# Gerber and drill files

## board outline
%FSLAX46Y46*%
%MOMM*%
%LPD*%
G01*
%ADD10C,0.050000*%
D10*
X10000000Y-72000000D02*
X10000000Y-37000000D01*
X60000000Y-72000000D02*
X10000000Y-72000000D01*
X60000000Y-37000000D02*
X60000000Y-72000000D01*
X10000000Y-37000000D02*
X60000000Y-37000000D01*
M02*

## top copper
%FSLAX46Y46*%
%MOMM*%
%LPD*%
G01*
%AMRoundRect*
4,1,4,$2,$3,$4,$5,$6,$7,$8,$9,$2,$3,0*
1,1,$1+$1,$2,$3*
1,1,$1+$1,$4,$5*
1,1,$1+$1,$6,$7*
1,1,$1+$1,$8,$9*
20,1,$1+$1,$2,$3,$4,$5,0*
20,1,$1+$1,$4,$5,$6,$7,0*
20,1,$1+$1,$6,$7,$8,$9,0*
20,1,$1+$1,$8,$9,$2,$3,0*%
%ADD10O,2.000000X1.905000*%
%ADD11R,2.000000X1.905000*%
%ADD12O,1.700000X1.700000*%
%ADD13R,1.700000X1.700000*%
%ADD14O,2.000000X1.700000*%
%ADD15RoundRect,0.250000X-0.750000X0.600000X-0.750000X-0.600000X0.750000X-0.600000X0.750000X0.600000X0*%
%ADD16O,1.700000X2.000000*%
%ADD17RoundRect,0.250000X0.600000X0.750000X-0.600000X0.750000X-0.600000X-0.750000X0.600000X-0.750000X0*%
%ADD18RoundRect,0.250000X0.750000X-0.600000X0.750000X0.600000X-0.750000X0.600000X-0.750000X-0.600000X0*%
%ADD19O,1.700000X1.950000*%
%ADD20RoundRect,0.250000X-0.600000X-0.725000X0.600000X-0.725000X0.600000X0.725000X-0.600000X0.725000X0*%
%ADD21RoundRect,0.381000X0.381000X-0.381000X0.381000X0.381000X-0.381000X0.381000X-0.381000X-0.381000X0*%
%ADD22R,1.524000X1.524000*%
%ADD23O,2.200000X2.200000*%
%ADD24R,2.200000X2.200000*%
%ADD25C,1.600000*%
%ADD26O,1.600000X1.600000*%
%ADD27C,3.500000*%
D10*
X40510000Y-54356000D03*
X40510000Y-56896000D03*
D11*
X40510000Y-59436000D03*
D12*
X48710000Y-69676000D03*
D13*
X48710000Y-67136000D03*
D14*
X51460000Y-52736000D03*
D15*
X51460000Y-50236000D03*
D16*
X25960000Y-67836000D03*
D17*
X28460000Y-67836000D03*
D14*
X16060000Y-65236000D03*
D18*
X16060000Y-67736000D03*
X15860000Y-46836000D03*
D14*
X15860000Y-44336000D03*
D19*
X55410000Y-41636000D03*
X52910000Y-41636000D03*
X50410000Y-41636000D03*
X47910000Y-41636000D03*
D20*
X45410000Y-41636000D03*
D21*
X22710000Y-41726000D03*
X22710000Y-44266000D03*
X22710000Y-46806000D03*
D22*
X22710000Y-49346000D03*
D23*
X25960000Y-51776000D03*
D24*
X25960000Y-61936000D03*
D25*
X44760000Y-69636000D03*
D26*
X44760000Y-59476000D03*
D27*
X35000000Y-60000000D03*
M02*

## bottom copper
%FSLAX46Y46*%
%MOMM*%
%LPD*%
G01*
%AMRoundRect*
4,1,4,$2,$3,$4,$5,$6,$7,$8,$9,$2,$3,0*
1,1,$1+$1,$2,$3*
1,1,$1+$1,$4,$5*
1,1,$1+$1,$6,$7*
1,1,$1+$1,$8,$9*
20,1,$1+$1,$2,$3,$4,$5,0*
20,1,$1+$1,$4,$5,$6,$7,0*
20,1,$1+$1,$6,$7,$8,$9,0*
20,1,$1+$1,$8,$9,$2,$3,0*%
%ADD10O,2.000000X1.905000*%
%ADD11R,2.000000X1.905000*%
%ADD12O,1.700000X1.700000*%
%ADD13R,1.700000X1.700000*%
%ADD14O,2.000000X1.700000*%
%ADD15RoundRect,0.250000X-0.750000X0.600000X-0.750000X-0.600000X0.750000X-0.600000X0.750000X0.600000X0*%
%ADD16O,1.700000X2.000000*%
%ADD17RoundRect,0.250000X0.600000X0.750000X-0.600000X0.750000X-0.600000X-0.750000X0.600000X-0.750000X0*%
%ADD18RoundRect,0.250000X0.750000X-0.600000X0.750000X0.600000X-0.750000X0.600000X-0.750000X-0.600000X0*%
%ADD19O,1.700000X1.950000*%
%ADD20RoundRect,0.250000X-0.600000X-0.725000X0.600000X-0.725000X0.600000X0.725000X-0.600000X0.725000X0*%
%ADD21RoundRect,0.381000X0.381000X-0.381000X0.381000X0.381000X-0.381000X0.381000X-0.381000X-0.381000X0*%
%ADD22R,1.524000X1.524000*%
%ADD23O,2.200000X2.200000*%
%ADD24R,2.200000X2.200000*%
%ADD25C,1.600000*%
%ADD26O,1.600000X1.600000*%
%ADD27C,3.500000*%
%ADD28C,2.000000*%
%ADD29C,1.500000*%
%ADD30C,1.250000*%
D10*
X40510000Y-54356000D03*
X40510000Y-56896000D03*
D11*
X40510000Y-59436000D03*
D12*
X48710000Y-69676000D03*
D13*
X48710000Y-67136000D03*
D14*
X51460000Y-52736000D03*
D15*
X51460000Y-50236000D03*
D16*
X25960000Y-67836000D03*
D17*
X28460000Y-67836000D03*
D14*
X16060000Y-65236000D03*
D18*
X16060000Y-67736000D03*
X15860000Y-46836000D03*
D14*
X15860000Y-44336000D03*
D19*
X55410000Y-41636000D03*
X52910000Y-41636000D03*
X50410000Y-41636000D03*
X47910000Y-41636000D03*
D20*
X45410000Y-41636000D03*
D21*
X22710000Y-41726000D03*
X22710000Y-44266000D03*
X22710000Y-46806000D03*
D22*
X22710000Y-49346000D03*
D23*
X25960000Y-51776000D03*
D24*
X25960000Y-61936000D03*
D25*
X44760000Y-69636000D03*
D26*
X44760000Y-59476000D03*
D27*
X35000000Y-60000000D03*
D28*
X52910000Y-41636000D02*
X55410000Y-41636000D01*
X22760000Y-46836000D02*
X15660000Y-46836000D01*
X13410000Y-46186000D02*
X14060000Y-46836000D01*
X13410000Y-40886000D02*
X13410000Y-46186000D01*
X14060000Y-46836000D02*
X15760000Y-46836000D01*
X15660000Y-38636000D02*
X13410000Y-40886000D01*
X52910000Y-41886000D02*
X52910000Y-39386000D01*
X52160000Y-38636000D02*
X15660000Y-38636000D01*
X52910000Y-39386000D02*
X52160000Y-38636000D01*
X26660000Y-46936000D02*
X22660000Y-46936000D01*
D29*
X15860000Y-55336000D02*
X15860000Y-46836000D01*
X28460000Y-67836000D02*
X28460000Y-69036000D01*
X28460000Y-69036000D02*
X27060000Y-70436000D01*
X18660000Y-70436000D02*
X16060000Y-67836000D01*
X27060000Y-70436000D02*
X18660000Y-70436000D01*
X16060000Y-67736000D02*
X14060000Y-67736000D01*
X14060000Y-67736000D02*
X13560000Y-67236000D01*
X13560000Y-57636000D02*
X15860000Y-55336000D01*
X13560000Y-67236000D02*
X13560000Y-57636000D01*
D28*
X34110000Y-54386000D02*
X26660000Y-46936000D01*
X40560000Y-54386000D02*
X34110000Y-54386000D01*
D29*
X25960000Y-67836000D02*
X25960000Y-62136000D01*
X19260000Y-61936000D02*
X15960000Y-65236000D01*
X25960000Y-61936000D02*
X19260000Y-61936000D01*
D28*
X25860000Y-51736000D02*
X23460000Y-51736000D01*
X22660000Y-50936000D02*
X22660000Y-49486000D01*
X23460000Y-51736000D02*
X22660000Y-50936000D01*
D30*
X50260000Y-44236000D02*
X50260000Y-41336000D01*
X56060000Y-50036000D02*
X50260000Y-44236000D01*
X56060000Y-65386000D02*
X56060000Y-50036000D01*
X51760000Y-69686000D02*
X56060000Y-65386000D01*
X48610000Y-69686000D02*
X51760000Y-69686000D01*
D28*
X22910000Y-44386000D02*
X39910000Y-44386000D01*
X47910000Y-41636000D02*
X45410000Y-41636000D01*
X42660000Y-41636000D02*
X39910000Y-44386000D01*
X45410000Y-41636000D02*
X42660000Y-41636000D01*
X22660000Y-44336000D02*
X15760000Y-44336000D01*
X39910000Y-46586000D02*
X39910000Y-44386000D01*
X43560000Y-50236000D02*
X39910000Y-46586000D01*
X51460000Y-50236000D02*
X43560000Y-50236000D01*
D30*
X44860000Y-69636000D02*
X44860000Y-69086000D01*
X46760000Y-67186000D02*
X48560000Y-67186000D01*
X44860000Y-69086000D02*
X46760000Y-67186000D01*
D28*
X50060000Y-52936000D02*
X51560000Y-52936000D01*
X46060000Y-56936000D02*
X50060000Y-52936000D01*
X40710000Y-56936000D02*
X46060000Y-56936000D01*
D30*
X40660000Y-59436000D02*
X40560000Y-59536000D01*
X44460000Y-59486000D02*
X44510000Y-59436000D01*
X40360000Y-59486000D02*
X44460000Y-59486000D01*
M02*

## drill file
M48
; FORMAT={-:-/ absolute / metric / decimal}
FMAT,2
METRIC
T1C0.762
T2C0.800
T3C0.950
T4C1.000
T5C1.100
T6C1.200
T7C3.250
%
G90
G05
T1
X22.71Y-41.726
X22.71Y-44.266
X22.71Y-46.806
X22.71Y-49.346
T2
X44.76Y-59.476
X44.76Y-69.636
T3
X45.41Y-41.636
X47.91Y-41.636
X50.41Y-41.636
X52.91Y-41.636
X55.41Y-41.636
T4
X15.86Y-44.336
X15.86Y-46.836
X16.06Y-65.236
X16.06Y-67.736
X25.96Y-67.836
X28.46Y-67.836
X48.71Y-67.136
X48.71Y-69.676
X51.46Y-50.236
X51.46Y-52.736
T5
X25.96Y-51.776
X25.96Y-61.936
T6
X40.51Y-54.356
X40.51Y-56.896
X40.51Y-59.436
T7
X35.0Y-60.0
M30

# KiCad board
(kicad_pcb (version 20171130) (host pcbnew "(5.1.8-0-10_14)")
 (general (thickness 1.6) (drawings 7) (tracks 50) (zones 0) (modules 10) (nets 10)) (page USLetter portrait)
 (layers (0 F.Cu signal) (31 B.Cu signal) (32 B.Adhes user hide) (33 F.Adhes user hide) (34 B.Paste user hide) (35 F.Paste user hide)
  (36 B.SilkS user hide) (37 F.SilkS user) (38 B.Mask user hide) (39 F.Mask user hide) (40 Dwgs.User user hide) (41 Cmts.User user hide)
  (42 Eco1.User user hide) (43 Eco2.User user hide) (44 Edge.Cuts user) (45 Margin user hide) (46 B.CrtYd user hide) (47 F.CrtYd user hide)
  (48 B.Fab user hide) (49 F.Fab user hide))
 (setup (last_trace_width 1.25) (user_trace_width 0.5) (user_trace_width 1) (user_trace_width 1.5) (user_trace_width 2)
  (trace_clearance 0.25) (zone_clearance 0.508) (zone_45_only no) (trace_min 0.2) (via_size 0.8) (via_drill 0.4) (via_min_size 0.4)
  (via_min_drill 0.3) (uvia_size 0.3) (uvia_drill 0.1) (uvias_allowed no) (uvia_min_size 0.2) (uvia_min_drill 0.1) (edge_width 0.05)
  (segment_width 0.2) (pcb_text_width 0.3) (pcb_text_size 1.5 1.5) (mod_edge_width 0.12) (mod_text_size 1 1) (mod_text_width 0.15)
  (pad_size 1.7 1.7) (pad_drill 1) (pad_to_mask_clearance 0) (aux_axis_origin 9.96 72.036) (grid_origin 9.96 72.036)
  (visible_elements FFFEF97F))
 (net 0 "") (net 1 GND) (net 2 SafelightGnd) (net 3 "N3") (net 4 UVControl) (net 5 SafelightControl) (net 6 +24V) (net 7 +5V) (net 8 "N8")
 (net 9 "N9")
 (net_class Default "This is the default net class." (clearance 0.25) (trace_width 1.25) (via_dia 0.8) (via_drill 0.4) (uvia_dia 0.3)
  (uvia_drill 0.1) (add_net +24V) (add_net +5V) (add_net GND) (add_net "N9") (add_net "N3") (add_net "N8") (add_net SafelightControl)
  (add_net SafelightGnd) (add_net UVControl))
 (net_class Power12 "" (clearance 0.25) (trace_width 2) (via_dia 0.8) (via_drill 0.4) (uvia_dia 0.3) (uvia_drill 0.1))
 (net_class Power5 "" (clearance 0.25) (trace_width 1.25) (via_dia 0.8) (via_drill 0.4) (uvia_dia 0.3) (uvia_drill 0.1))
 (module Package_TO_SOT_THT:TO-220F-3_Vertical (layer F.Cu) (at 40.51 59.436 90)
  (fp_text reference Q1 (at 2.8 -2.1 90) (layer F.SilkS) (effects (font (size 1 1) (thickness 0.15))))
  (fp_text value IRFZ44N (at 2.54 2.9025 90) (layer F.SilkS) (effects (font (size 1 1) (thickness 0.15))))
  (pad 3 thru_hole oval (at 5.08 0 90) (size 1.905 2) (drill 1.2) (layers *.Cu *.Mask) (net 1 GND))
  (pad 2 thru_hole oval (at 2.54 0 90) (size 1.905 2) (drill 1.2) (layers *.Cu *.Mask) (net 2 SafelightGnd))
  (pad 1 thru_hole rect (at 0 0 90) (size 1.905 2) (drill 1.2) (layers *.Cu *.Mask) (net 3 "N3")))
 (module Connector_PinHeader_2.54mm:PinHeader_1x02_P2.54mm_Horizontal (layer F.Cu) (at 48.71 67.136)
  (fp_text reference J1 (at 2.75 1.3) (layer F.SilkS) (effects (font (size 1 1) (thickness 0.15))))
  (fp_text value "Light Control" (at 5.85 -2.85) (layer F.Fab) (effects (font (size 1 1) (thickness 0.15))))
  (pad 2 thru_hole oval (at 0 2.54) (size 1.7 1.7) (drill 1) (layers *.Cu *.Mask) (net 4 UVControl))
  (pad 1 thru_hole rect (at 0 0) (size 1.7 1.7) (drill 1) (layers *.Cu *.Mask) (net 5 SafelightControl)))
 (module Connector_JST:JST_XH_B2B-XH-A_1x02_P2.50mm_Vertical (layer F.Cu) (at 51.46 50.236 270)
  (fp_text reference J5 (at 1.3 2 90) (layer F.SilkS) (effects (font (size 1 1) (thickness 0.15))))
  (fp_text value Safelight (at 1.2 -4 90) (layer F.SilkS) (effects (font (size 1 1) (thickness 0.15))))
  (pad 2 thru_hole oval (at 2.5 0 270) (size 1.7 2) (drill 1) (layers *.Cu *.Mask) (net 2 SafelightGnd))
  (pad 1 thru_hole roundrect (at 0 0 270) (size 1.7 2) (drill 1) (layers *.Cu *.Mask) (roundrect_rratio 0.1470588235294118) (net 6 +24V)))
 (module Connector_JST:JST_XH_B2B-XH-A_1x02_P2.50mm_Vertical (layer F.Cu) (at 28.46 67.836 180)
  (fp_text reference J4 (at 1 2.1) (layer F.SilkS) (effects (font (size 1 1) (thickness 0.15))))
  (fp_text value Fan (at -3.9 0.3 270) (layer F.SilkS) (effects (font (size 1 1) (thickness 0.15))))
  (pad 2 thru_hole oval (at 2.5 0 180) (size 1.7 2) (drill 1) (layers *.Cu *.Mask) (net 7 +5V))
  (pad 1 thru_hole roundrect (at 0 0 180) (size 1.7 2) (drill 1) (layers *.Cu *.Mask) (roundrect_rratio 0.1470588235294118) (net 1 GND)))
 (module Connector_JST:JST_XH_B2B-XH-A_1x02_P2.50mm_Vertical (layer F.Cu) (at 16.06 67.736 90)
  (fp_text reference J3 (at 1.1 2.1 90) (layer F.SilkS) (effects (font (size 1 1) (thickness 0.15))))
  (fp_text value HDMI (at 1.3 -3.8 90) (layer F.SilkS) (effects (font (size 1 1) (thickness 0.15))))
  (pad 2 thru_hole oval (at 2.5 0 90) (size 1.7 2) (drill 1) (layers *.Cu *.Mask) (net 7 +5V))
  (pad 1 thru_hole roundrect (at 0 0 90) (size 1.7 2) (drill 1) (layers *.Cu *.Mask) (roundrect_rratio 0.1470588235294118) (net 1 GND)))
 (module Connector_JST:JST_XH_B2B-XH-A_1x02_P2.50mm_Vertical (layer F.Cu) (at 15.86 46.836 90)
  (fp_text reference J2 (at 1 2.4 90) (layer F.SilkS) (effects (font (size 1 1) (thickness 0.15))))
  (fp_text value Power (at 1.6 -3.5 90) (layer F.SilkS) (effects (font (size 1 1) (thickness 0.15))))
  (pad 1 thru_hole roundrect (at 0 0 90) (size 1.7 2) (drill 1) (layers *.Cu *.Mask) (roundrect_rratio 0.1470588235294118) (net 1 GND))
  (pad 2 thru_hole oval (at 2.5 0 90) (size 1.7 2) (drill 1) (layers *.Cu *.Mask) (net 6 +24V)))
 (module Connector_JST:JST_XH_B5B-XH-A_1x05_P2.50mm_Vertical (layer F.Cu) (at 45.41 41.636)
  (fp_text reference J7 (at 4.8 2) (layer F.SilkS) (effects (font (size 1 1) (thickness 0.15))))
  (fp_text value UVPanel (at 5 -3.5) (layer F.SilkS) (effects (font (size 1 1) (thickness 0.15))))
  (pad 5 thru_hole oval (at 10 0) (size 1.7 1.95) (drill 0.95) (layers *.Cu *.Mask) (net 1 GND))
  (pad 4 thru_hole oval (at 7.5 0) (size 1.7 1.95) (drill 0.95) (layers *.Cu *.Mask) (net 1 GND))
  (pad 3 thru_hole oval (at 5 0) (size 1.7 1.95) (drill 0.95) (layers *.Cu *.Mask) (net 4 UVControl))
  (pad 2 thru_hole oval (at 2.5 0) (size 1.7 1.95) (drill 0.95) (layers *.Cu *.Mask) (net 6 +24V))
  (pad 1 thru_hole roundrect (at 0 0) (size 1.7 1.95) (drill 0.95) (layers *.Cu *.Mask) (roundrect_rratio 0.1470588235294118) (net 6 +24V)))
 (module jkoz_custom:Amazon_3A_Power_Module (layer F.Cu) (at 30.66 45.636 90)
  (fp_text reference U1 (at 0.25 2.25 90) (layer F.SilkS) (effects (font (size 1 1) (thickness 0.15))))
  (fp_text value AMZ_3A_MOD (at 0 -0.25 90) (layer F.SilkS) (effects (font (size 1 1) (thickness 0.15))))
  (pad 4 thru_hole roundrect (at 3.91 -7.95 90) (size 1.524 1.524) (drill 0.762) (layers *.Cu *.Mask) (roundrect_rratio 0.25) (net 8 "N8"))
  (pad 3 thru_hole roundrect (at 1.37 -7.95 90) (size 1.524 1.524) (drill 0.762) (layers *.Cu *.Mask) (roundrect_rratio 0.25) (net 6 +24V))
  (pad 2 thru_hole roundrect (at -1.17 -7.95 90) (size 1.524 1.524) (drill 0.762) (layers *.Cu *.Mask) (roundrect_rratio 0.25) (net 1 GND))
  (pad 1 thru_hole rect (at -3.71 -7.95 90) (size 1.524 1.524) (drill 0.762) (layers *.Cu *.Mask) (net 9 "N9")))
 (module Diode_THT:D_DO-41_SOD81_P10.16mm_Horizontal (layer F.Cu) (at 25.96 61.936 90)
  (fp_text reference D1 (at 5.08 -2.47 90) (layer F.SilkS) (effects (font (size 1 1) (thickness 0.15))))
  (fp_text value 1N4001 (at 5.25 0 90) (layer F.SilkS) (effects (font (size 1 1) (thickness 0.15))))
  (pad 2 thru_hole oval (at 10.16 0 90) (size 2.2 2.2) (drill 1.1) (layers *.Cu *.Mask) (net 9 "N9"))
  (pad 1 thru_hole rect (at 0 0 90) (size 2.2 2.2) (drill 1.1) (layers *.Cu *.Mask) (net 7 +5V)))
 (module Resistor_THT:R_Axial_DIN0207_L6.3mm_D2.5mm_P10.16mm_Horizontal (layer F.Cu) (at 44.76 69.636 90)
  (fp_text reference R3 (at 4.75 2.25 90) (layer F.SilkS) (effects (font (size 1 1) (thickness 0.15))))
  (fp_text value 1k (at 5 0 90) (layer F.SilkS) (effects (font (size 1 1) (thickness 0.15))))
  (pad 1 thru_hole circle (at 0 0 90) (size 1.6 1.6) (drill 0.8) (layers *.Cu *.Mask) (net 5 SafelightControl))
  (pad 2 thru_hole oval (at 10.16 0 90) (size 1.6 1.6) (drill 0.8) (layers *.Cu *.Mask) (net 3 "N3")))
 (gr_line (start 10 72) (end 10 37) (layer Edge.Cuts) (width 0.05))
 (gr_line (start 60 72) (end 10 72) (layer Edge.Cuts) (width 0.05))
 (gr_line (start 60 37) (end 60 72) (layer Edge.Cuts) (width 0.05))
 (gr_line (start 10 37) (end 60 37) (layer Edge.Cuts) (width 0.05))
 (via (at 35 60) (size 3.5) (drill 3.25) (layers F.Cu B.Cu) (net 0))
 (segment (start 52.91 41.636) (end 55.41 41.636) (width 2) (layer B.Cu) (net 1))
 (segment (start 22.76 46.836) (end 15.66 46.836) (width 2) (layer B.Cu) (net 1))
 (segment (start 13.41 46.186) (end 14.06 46.836) (width 2) (layer B.Cu) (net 1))
 (segment (start 13.41 40.886) (end 13.41 46.186) (width 2) (layer B.Cu) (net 1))
 (segment (start 14.06 46.836) (end 15.76 46.836) (width 2) (layer B.Cu) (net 1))
 (segment (start 15.66 38.636) (end 13.41 40.886) (width 2) (layer B.Cu) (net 1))
 (segment (start 52.91 41.886) (end 52.91 39.386) (width 2) (layer B.Cu) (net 1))
 (segment (start 52.16 38.636) (end 15.66 38.636) (width 2) (layer B.Cu) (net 1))
 (segment (start 52.91 39.386) (end 52.16 38.636) (width 2) (layer B.Cu) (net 1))
 (segment (start 26.66 46.936) (end 22.66 46.936) (width 2) (layer B.Cu) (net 1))
 (segment (start 15.86 55.336) (end 15.86 46.836) (width 1.5) (layer B.Cu) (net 1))
 (segment (start 28.46 67.836) (end 28.46 69.036) (width 1.5) (layer B.Cu) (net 1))
 (segment (start 28.46 69.036) (end 27.06 70.436) (width 1.5) (layer B.Cu) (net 1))
 (segment (start 18.66 70.436) (end 16.06 67.836) (width 1.5) (layer B.Cu) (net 1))
 (segment (start 27.06 70.436) (end 18.66 70.436) (width 1.5) (layer B.Cu) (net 1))
 (segment (start 16.06 67.736) (end 14.06 67.736) (width 1.5) (layer B.Cu) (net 1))
 (segment (start 14.06 67.736) (end 13.56 67.236) (width 1.5) (layer B.Cu) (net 1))
 (segment (start 13.56 57.636) (end 15.86 55.336) (width 1.5) (layer B.Cu) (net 1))
 (segment (start 13.56 67.236) (end 13.56 57.636) (width 1.5) (layer B.Cu) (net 1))
 (segment (start 34.11 54.386) (end 26.66 46.936) (width 2) (layer B.Cu) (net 1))
 (segment (start 40.56 54.386) (end 34.11 54.386) (width 2) (layer B.Cu) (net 1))
 (segment (start 25.96 67.836) (end 25.96 62.136) (width 1.5) (layer B.Cu) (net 7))
 (segment (start 19.26 61.936) (end 15.96 65.236) (width 1.5) (layer B.Cu) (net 7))
 (segment (start 25.96 61.936) (end 19.26 61.936) (width 1.5) (layer B.Cu) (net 7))
 (segment (start 25.86 51.736) (end 23.46 51.736) (width 2) (layer B.Cu) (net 9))
 (segment (start 22.66 50.936) (end 22.66 49.486) (width 2) (layer B.Cu) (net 9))
 (segment (start 23.46 51.736) (end 22.66 50.936) (width 2) (layer B.Cu) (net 9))
 (segment (start 50.26 44.236) (end 50.26 41.336) (width 1.25) (layer B.Cu) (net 4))
 (segment (start 56.06 50.036) (end 50.26 44.236) (width 1.25) (layer B.Cu) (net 4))
 (segment (start 56.06 65.386) (end 56.06 50.036) (width 1.25) (layer B.Cu) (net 4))
 (segment (start 51.76 69.686) (end 56.06 65.386) (width 1.25) (layer B.Cu) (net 4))
 (segment (start 48.61 69.686) (end 51.76 69.686) (width 1.25) (layer B.Cu) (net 4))
 (segment (start 22.91 44.386) (end 39.91 44.386) (width 2) (layer B.Cu) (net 6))
 (segment (start 47.91 41.636) (end 45.41 41.636) (width 2) (layer B.Cu) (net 6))
 (segment (start 42.66 41.636) (end 39.91 44.386) (width 2) (layer B.Cu) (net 6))
 (segment (start 45.41 41.636) (end 42.66 41.636) (width 2) (layer B.Cu) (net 6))
 (segment (start 22.66 44.336) (end 15.76 44.336) (width 2) (layer B.Cu) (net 6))
 (segment (start 39.91 46.586) (end 39.91 44.386) (width 2) (layer B.Cu) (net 6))
 (segment (start 43.56 50.236) (end 39.91 46.586) (width 2) (layer B.Cu) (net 6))
 (segment (start 51.46 50.236) (end 43.56 50.236) (width 2) (layer B.Cu) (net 6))
 (segment (start 44.86 69.636) (end 44.86 69.086) (width 1.25) (layer B.Cu) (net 5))
 (segment (start 46.76 67.186) (end 48.56 67.186) (width 1.25) (layer B.Cu) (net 5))
 (segment (start 44.86 69.086) (end 46.76 67.186) (width 1.25) (layer B.Cu) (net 5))
 (segment (start 50.06 52.936) (end 51.56 52.936) (width 2) (layer B.Cu) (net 2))
 (segment (start 46.06 56.936) (end 50.06 52.936) (width 2) (layer B.Cu) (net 2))
 (segment (start 40.71 56.936) (end 46.06 56.936) (width 2) (layer B.Cu) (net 2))
 (segment (start 40.66 59.436) (end 40.56 59.536) (width 1.25) (layer B.Cu) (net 3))
 (segment (start 44.46 59.486) (end 44.51 59.436) (width 1.25) (layer B.Cu) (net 3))
 (segment (start 40.36 59.486) (end 44.46 59.486) (width 1.25) (layer B.Cu) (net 3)))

